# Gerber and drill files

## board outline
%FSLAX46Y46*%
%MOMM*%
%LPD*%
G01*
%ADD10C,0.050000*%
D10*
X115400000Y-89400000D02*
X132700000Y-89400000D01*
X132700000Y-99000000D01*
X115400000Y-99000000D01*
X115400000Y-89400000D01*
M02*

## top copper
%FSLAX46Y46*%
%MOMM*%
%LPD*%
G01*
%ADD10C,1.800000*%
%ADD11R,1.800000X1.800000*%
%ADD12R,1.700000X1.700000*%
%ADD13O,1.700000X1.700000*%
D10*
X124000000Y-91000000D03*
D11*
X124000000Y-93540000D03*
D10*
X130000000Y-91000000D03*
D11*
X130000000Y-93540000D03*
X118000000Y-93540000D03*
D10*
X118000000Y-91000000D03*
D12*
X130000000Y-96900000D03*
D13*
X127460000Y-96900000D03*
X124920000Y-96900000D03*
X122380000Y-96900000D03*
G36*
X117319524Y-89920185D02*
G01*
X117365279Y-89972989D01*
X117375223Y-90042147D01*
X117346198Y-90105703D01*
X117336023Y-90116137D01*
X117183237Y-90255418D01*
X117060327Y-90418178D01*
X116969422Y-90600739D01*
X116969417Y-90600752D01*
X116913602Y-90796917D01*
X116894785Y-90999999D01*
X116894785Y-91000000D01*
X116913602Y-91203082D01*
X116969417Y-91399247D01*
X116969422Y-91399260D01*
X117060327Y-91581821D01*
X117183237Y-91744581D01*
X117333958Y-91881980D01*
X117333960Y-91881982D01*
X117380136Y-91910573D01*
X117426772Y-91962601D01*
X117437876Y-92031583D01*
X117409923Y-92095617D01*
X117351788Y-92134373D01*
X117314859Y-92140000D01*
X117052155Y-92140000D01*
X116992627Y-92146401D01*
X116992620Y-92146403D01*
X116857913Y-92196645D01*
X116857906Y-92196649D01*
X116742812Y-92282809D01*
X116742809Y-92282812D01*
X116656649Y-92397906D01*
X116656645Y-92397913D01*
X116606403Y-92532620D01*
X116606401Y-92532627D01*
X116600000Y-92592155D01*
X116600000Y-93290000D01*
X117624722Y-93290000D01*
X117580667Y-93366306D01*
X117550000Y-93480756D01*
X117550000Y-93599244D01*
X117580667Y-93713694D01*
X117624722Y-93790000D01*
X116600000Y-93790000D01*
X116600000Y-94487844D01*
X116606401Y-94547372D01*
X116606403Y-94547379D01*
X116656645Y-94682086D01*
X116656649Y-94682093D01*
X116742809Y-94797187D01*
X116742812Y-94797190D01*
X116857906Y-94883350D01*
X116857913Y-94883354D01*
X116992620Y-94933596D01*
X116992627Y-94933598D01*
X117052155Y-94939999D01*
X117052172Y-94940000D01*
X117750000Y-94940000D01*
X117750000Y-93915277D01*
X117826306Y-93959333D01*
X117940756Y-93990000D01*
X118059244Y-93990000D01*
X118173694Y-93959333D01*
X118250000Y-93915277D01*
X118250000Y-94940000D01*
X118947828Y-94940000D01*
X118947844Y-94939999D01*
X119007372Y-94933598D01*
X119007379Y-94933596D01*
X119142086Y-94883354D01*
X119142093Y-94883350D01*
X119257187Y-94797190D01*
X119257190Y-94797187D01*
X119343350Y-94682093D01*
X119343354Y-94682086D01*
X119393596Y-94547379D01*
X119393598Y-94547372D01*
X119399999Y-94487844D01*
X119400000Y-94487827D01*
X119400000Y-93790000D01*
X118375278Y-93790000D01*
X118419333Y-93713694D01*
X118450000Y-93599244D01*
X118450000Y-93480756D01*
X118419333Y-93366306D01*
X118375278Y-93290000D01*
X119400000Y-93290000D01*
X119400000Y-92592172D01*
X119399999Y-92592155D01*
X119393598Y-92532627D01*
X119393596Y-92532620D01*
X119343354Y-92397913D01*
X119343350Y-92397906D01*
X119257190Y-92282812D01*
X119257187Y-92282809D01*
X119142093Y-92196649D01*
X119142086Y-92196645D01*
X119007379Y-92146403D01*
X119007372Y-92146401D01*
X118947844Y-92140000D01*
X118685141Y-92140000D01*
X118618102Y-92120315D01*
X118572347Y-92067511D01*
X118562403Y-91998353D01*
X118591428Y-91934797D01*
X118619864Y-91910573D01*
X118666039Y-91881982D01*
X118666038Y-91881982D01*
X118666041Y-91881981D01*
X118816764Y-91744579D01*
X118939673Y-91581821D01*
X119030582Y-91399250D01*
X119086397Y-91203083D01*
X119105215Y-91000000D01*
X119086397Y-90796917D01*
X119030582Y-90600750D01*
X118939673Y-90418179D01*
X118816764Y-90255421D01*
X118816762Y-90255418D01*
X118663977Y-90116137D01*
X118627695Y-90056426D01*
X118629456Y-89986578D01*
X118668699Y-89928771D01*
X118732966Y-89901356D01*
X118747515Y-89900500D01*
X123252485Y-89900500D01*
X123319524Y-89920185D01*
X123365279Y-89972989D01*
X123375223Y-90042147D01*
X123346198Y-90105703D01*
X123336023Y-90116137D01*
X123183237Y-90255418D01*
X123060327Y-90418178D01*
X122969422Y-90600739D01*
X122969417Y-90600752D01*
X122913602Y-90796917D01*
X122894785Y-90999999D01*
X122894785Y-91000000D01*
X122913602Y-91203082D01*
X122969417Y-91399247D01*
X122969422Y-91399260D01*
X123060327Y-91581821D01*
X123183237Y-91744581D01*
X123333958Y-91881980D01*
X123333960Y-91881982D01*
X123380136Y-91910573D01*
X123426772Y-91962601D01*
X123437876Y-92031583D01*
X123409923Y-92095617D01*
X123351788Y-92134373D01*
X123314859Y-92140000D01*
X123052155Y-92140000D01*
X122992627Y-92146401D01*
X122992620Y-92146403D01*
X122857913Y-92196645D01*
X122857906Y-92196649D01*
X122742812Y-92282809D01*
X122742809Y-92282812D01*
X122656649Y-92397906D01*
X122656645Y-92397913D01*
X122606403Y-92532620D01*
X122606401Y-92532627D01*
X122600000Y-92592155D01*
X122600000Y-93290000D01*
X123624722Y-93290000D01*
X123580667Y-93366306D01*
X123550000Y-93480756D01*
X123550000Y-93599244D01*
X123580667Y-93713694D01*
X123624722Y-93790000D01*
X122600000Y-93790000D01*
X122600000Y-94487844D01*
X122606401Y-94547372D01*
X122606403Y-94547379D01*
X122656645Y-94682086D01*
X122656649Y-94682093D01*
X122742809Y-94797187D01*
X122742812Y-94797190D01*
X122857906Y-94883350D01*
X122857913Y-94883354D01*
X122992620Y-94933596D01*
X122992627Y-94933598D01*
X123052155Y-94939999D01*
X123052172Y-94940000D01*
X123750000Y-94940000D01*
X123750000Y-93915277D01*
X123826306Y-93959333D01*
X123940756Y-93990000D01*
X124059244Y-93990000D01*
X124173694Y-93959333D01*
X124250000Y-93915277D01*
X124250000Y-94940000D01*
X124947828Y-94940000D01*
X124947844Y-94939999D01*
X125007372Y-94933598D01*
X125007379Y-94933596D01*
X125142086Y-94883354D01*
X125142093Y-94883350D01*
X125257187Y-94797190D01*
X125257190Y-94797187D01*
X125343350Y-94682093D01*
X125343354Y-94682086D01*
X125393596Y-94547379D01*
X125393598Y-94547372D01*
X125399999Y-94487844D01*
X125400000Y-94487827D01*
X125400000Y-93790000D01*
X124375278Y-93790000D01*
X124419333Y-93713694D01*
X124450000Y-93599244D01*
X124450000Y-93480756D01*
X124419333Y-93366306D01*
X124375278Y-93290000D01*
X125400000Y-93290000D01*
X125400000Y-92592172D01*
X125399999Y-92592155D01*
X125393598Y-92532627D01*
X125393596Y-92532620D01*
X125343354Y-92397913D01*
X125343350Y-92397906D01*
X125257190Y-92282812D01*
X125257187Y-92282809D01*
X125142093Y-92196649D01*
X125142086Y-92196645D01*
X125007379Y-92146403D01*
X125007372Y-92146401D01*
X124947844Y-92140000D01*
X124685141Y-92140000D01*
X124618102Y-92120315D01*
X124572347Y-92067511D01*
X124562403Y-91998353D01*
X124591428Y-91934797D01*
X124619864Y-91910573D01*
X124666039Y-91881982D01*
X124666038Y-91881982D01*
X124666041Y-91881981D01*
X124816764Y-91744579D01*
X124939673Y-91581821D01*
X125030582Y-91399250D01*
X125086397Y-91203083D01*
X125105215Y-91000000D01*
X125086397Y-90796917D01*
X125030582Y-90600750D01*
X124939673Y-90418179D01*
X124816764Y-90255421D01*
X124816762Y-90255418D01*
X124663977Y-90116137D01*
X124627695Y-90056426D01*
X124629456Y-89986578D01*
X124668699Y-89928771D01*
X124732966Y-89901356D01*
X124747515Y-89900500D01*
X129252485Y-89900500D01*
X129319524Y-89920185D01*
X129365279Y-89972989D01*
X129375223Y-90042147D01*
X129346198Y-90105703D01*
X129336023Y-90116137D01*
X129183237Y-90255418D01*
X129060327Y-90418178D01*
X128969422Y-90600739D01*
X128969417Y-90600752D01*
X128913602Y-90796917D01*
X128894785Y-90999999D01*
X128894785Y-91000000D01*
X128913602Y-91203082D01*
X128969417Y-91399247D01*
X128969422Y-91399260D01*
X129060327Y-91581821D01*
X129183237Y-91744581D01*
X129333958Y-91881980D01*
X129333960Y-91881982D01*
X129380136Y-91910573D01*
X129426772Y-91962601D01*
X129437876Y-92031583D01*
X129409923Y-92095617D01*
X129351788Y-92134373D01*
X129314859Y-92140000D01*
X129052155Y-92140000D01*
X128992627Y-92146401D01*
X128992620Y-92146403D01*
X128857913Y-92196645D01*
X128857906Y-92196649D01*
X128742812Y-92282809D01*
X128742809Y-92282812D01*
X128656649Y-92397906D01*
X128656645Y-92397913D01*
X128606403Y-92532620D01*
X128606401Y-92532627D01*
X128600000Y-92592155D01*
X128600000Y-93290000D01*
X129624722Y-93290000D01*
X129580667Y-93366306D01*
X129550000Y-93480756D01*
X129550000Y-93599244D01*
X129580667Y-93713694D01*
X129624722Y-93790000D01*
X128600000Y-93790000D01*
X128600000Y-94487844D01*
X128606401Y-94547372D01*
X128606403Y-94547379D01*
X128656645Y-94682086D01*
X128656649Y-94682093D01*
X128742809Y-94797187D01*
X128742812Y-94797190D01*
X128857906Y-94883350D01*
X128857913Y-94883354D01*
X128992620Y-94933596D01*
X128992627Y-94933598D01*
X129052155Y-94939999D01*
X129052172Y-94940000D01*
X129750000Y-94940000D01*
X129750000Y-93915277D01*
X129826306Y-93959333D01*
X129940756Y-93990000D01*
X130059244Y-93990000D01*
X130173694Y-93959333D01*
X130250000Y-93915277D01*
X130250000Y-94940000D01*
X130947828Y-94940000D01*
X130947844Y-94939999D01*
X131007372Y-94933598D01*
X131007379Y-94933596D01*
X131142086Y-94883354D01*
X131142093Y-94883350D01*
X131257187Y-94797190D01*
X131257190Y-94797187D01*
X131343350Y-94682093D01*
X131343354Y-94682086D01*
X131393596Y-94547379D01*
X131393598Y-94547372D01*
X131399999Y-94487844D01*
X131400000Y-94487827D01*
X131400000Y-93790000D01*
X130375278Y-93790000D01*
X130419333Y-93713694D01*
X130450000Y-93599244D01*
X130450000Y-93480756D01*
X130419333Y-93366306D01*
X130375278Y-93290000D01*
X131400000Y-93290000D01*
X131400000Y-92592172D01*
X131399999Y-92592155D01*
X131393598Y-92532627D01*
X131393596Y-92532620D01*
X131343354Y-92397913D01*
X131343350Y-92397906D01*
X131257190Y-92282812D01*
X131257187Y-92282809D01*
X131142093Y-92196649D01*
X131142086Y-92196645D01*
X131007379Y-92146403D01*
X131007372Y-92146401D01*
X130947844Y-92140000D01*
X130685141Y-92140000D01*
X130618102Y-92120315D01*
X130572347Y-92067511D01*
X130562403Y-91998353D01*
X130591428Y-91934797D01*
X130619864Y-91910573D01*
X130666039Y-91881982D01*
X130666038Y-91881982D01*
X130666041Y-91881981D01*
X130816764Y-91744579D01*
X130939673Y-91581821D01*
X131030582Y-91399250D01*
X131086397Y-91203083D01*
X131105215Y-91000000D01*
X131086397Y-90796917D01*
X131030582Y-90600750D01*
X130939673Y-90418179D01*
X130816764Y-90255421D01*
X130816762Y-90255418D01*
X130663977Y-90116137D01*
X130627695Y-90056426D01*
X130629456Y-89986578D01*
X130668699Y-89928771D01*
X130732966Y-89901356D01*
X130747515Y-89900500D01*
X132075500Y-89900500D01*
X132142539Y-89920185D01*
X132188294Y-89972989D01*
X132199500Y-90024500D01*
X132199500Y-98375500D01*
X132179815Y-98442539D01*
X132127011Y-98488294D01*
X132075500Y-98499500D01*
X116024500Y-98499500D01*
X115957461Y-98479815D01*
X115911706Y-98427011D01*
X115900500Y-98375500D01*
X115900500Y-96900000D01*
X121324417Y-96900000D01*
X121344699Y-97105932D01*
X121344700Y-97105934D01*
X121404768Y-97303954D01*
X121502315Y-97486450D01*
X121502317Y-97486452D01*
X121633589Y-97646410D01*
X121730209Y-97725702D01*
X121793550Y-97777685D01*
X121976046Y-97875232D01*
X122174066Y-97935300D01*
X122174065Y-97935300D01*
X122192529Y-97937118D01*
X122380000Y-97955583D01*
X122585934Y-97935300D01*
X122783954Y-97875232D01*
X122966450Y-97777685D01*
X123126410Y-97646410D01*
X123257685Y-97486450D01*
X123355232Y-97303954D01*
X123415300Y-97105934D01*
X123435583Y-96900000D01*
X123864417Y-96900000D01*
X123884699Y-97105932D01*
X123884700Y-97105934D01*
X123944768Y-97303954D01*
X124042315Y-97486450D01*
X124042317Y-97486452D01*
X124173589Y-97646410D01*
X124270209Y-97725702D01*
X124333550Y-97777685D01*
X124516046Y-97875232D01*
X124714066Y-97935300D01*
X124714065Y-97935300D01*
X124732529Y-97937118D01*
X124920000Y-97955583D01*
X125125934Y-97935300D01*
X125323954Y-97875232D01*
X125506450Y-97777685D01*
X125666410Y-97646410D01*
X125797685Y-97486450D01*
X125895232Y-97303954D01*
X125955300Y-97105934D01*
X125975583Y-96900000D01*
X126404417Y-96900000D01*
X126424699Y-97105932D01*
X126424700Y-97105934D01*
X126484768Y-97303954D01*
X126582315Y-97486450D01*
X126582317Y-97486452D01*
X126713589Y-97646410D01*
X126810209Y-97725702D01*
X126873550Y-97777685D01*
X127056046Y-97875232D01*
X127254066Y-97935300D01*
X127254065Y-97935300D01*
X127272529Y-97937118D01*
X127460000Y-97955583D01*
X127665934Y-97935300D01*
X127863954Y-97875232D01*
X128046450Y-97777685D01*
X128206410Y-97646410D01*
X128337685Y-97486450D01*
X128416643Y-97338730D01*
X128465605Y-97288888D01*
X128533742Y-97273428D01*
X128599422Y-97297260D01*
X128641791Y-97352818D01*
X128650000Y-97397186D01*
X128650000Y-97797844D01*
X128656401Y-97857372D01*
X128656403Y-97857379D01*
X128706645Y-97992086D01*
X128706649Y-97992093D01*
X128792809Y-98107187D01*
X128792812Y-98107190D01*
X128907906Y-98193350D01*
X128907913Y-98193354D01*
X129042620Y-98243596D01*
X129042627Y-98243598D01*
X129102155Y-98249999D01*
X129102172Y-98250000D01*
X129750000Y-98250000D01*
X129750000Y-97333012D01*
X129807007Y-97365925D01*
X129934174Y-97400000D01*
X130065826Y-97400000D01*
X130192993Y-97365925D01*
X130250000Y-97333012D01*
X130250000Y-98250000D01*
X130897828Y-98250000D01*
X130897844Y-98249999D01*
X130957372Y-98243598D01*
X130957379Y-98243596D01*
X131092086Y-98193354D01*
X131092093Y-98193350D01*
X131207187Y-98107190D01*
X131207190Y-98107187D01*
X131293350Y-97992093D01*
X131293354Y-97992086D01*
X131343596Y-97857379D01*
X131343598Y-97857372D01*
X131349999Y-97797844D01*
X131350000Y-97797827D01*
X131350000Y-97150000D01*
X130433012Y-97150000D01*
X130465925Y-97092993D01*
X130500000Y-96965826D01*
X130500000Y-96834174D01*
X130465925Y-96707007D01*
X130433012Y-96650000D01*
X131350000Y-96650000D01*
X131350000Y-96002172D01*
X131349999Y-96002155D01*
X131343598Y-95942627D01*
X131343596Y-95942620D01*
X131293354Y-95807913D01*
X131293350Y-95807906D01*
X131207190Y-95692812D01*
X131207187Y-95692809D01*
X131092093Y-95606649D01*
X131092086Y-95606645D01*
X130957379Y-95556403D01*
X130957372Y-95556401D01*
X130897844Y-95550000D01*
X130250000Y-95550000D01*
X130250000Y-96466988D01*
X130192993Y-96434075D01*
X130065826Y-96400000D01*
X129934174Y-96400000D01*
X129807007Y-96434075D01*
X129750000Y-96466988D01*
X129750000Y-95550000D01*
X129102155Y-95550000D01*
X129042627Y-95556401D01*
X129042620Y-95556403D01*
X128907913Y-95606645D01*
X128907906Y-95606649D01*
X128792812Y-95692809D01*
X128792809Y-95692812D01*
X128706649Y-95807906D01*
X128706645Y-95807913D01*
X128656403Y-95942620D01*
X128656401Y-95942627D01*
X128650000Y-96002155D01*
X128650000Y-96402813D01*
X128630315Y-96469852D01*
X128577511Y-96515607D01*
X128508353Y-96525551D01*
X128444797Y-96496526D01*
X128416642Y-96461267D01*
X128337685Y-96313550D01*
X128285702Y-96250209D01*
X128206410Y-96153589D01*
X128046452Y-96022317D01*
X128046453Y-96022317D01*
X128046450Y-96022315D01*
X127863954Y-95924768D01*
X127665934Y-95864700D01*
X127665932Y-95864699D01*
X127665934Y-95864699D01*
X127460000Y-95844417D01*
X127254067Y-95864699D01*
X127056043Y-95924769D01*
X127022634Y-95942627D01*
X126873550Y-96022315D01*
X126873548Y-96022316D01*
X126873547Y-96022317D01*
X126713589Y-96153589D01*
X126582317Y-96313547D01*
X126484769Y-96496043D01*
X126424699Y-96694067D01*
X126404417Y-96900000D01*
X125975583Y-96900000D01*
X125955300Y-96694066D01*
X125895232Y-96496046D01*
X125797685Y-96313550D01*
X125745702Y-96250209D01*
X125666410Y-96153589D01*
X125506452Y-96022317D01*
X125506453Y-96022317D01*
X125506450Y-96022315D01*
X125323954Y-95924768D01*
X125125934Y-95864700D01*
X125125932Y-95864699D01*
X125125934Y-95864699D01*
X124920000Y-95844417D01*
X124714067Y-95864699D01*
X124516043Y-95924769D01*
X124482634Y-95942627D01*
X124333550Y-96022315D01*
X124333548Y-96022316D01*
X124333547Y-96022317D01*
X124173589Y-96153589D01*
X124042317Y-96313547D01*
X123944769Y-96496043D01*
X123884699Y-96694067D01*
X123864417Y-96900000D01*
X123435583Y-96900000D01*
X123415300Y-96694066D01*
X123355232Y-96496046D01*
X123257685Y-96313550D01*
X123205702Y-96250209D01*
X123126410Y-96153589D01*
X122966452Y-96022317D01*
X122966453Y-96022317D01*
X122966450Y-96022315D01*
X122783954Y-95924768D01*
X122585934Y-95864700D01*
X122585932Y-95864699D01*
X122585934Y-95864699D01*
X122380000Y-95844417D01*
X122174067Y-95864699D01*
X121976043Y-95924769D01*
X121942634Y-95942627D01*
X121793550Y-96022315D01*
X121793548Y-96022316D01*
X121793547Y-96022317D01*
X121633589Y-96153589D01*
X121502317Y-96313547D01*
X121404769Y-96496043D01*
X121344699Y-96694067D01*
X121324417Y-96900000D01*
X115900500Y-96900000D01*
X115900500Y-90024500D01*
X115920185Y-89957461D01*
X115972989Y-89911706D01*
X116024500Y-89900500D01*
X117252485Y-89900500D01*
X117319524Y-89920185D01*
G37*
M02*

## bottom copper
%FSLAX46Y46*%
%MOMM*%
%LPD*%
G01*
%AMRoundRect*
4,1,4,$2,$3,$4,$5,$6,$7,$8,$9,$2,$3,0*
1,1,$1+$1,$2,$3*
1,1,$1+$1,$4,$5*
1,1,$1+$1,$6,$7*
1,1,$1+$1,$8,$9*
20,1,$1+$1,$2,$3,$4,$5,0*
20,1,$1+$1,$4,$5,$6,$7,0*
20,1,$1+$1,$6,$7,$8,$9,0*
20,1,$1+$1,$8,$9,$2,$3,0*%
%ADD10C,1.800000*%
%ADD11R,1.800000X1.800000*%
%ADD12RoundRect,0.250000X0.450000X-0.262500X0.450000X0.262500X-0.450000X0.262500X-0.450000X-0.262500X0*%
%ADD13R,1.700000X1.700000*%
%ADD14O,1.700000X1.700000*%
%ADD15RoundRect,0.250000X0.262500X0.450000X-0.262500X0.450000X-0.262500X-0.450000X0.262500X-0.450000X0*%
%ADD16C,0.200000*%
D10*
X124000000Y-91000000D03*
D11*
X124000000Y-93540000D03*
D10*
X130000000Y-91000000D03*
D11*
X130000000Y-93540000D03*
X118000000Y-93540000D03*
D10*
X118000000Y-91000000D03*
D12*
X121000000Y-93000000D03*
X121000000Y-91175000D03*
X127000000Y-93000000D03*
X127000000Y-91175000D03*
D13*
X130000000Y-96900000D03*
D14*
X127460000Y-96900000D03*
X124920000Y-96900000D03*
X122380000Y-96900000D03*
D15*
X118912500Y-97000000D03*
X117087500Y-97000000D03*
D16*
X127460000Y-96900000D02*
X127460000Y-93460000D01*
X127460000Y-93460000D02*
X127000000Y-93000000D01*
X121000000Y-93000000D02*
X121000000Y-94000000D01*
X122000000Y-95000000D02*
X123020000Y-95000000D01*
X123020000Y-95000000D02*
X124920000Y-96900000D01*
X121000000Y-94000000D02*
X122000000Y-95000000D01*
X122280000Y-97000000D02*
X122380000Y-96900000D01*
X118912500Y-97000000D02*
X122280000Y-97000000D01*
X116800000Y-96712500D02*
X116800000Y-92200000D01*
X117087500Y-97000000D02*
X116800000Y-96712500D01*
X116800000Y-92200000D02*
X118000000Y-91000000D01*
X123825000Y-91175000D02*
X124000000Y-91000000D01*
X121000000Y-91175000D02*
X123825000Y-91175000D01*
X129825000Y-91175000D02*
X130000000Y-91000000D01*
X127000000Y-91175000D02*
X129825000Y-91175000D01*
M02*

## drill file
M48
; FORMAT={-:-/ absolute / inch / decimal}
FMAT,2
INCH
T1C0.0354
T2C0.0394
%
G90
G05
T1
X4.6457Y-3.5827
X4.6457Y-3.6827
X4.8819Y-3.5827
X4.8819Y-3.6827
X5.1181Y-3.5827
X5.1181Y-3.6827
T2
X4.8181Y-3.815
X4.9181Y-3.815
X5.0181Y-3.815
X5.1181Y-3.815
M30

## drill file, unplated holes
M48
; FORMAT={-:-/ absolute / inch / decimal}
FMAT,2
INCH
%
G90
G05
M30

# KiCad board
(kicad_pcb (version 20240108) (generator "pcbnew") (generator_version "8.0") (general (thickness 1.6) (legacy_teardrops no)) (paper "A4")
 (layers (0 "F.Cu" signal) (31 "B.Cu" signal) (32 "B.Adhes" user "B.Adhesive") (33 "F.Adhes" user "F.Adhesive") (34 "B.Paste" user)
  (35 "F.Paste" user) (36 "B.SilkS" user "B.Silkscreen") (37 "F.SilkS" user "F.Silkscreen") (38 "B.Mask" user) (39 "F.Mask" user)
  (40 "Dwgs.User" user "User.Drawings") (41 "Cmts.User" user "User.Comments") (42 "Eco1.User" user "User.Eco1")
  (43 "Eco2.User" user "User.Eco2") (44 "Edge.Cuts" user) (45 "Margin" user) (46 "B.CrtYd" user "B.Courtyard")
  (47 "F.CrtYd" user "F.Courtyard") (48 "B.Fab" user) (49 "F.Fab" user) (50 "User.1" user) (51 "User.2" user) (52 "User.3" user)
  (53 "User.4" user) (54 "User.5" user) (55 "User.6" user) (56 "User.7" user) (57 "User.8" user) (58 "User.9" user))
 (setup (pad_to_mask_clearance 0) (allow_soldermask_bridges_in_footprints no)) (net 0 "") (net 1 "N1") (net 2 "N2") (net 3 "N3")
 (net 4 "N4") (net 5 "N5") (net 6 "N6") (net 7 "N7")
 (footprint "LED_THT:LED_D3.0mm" (layer "F.Cu") (at 124 93.54 90)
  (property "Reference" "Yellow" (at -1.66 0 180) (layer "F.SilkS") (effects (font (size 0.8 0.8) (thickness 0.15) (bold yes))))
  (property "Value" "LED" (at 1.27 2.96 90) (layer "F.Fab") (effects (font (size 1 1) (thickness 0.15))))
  (pad "1" thru_hole rect (at 0 0 90) (size 1.8 1.8) (drill 0.9) (layers "*.Cu" "*.Mask") (remove_unused_layers no) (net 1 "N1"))
  (pad "2" thru_hole circle (at 2.54 0 90) (size 1.8 1.8) (drill 0.9) (layers "*.Cu" "*.Mask") (remove_unused_layers no) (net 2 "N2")))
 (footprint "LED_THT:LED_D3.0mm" (layer "F.Cu") (at 130 93.54 90)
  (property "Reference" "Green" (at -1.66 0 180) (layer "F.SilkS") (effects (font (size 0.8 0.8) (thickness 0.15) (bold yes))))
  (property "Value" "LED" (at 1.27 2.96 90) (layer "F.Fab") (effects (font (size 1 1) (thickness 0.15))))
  (pad "1" thru_hole rect (at 0 0 90) (size 1.8 1.8) (drill 0.9) (layers "*.Cu" "*.Mask") (remove_unused_layers no) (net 1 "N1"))
  (pad "2" thru_hole circle (at 2.54 0 90) (size 1.8 1.8) (drill 0.9) (layers "*.Cu" "*.Mask") (remove_unused_layers no) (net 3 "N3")))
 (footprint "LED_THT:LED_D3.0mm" (layer "F.Cu") (at 118 93.54 90)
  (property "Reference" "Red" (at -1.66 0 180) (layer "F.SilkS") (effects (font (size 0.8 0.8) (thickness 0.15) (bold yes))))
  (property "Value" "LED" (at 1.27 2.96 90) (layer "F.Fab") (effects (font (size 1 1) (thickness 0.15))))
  (pad "1" thru_hole rect (at 0 0 90) (size 1.8 1.8) (drill 0.9) (layers "*.Cu" "*.Mask") (remove_unused_layers no) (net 1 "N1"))
  (pad "2" thru_hole circle (at 2.54 0 90) (size 1.8 1.8) (drill 0.9) (layers "*.Cu" "*.Mask") (remove_unused_layers no) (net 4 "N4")))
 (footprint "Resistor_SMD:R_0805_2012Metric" (layer "B.Cu") (at 121 92.0875 90)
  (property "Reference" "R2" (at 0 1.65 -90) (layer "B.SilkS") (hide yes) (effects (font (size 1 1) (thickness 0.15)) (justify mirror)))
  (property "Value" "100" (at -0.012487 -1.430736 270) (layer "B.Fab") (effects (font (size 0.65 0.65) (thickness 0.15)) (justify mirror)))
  (pad "1" smd roundrect (at -0.9125 0 90) (size 1.025 1.4) (layers "B.Cu" "B.Paste" "B.Mask") (roundrect_rratio 0.243902) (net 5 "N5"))
  (pad "2" smd roundrect (at 0.9125 0 90) (size 1.025 1.4) (layers "B.Cu" "B.Paste" "B.Mask") (roundrect_rratio 0.243902) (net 2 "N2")))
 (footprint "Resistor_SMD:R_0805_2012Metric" (layer "B.Cu") (at 127 92.0875 90)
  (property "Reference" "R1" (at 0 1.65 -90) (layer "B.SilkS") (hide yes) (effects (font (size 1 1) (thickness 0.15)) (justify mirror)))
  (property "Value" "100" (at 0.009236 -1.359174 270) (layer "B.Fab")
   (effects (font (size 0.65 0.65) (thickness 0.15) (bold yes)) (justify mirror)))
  (pad "1" smd roundrect (at -0.9125 0 90) (size 1.025 1.4) (layers "B.Cu" "B.Paste" "B.Mask") (roundrect_rratio 0.243902) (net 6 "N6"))
  (pad "2" smd roundrect (at 0.9125 0 90) (size 1.025 1.4) (layers "B.Cu" "B.Paste" "B.Mask") (roundrect_rratio 0.243902) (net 3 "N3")))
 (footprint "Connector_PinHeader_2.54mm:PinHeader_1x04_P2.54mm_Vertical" (layer "B.Cu") (at 130 96.9 90)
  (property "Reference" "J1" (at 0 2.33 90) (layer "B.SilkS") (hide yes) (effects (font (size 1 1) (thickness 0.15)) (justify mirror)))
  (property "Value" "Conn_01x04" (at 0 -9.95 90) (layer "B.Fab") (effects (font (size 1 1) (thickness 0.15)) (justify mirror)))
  (pad "1" thru_hole rect (at 0 0 90) (size 1.7 1.7) (drill 1) (layers "*.Cu" "*.Mask") (remove_unused_layers no) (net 1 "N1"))
  (pad "2" thru_hole oval (at 0 -2.54 90) (size 1.7 1.7) (drill 1) (layers "*.Cu" "*.Mask") (remove_unused_layers no) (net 6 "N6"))
  (pad "3" thru_hole oval (at 0 -5.08 90) (size 1.7 1.7) (drill 1) (layers "*.Cu" "*.Mask") (remove_unused_layers no) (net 5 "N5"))
  (pad "4" thru_hole oval (at 0 -7.62 90) (size 1.7 1.7) (drill 1) (layers "*.Cu" "*.Mask") (remove_unused_layers no) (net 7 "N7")))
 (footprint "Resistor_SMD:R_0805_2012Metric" (layer "B.Cu") (at 118 97 180)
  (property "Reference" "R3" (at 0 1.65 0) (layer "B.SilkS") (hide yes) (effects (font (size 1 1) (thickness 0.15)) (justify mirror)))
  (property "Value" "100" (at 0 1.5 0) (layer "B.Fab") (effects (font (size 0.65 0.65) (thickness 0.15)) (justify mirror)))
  (pad "1" smd roundrect (at -0.9125 0 180) (size 1.025 1.4) (layers "B.Cu" "B.Paste" "B.Mask") (roundrect_rratio 0.243902) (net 7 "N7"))
  (pad "2" smd roundrect (at 0.9125 0 180) (size 1.025 1.4) (layers "B.Cu" "B.Paste" "B.Mask") (roundrect_rratio 0.243902) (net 4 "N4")))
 (gr_rect (start 115.4 89.4) (end 132.7 99) (stroke (width 0.05) (type default)) (fill none) (layer "Edge.Cuts"))
 (segment (start 127.46 96.9) (end 127.46 93.46) (width 0.2) (layer "B.Cu") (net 6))
 (segment (start 127.46 93.46) (end 127 93) (width 0.2) (layer "B.Cu") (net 6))
 (segment (start 121 93) (end 121 94) (width 0.2) (layer "B.Cu") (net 5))
 (segment (start 122 95) (end 123.02 95) (width 0.2) (layer "B.Cu") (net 5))
 (segment (start 123.02 95) (end 124.92 96.9) (width 0.2) (layer "B.Cu") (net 5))
 (segment (start 121 94) (end 122 95) (width 0.2) (layer "B.Cu") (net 5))
 (segment (start 122.28 97) (end 122.38 96.9) (width 0.2) (layer "B.Cu") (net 7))
 (segment (start 118.9125 97) (end 122.28 97) (width 0.2) (layer "B.Cu") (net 7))
 (segment (start 116.8 96.7125) (end 116.8 92.2) (width 0.2) (layer "B.Cu") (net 4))
 (segment (start 117.0875 97) (end 116.8 96.7125) (width 0.2) (layer "B.Cu") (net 4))
 (segment (start 116.8 92.2) (end 118 91) (width 0.2) (layer "B.Cu") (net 4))
 (segment (start 123.825 91.175) (end 124 91) (width 0.2) (layer "B.Cu") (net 2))
 (segment (start 121 91.175) (end 123.825 91.175) (width 0.2) (layer "B.Cu") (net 2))
 (segment (start 129.825 91.175) (end 130 91) (width 0.2) (layer "B.Cu") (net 3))
 (segment (start 127 91.175) (end 129.825 91.175) (width 0.2) (layer "B.Cu") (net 3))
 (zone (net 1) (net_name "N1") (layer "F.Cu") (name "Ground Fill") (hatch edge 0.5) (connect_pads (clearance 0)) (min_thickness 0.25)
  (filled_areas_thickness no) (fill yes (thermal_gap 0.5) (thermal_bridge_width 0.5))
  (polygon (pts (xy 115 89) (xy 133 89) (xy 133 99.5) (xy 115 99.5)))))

